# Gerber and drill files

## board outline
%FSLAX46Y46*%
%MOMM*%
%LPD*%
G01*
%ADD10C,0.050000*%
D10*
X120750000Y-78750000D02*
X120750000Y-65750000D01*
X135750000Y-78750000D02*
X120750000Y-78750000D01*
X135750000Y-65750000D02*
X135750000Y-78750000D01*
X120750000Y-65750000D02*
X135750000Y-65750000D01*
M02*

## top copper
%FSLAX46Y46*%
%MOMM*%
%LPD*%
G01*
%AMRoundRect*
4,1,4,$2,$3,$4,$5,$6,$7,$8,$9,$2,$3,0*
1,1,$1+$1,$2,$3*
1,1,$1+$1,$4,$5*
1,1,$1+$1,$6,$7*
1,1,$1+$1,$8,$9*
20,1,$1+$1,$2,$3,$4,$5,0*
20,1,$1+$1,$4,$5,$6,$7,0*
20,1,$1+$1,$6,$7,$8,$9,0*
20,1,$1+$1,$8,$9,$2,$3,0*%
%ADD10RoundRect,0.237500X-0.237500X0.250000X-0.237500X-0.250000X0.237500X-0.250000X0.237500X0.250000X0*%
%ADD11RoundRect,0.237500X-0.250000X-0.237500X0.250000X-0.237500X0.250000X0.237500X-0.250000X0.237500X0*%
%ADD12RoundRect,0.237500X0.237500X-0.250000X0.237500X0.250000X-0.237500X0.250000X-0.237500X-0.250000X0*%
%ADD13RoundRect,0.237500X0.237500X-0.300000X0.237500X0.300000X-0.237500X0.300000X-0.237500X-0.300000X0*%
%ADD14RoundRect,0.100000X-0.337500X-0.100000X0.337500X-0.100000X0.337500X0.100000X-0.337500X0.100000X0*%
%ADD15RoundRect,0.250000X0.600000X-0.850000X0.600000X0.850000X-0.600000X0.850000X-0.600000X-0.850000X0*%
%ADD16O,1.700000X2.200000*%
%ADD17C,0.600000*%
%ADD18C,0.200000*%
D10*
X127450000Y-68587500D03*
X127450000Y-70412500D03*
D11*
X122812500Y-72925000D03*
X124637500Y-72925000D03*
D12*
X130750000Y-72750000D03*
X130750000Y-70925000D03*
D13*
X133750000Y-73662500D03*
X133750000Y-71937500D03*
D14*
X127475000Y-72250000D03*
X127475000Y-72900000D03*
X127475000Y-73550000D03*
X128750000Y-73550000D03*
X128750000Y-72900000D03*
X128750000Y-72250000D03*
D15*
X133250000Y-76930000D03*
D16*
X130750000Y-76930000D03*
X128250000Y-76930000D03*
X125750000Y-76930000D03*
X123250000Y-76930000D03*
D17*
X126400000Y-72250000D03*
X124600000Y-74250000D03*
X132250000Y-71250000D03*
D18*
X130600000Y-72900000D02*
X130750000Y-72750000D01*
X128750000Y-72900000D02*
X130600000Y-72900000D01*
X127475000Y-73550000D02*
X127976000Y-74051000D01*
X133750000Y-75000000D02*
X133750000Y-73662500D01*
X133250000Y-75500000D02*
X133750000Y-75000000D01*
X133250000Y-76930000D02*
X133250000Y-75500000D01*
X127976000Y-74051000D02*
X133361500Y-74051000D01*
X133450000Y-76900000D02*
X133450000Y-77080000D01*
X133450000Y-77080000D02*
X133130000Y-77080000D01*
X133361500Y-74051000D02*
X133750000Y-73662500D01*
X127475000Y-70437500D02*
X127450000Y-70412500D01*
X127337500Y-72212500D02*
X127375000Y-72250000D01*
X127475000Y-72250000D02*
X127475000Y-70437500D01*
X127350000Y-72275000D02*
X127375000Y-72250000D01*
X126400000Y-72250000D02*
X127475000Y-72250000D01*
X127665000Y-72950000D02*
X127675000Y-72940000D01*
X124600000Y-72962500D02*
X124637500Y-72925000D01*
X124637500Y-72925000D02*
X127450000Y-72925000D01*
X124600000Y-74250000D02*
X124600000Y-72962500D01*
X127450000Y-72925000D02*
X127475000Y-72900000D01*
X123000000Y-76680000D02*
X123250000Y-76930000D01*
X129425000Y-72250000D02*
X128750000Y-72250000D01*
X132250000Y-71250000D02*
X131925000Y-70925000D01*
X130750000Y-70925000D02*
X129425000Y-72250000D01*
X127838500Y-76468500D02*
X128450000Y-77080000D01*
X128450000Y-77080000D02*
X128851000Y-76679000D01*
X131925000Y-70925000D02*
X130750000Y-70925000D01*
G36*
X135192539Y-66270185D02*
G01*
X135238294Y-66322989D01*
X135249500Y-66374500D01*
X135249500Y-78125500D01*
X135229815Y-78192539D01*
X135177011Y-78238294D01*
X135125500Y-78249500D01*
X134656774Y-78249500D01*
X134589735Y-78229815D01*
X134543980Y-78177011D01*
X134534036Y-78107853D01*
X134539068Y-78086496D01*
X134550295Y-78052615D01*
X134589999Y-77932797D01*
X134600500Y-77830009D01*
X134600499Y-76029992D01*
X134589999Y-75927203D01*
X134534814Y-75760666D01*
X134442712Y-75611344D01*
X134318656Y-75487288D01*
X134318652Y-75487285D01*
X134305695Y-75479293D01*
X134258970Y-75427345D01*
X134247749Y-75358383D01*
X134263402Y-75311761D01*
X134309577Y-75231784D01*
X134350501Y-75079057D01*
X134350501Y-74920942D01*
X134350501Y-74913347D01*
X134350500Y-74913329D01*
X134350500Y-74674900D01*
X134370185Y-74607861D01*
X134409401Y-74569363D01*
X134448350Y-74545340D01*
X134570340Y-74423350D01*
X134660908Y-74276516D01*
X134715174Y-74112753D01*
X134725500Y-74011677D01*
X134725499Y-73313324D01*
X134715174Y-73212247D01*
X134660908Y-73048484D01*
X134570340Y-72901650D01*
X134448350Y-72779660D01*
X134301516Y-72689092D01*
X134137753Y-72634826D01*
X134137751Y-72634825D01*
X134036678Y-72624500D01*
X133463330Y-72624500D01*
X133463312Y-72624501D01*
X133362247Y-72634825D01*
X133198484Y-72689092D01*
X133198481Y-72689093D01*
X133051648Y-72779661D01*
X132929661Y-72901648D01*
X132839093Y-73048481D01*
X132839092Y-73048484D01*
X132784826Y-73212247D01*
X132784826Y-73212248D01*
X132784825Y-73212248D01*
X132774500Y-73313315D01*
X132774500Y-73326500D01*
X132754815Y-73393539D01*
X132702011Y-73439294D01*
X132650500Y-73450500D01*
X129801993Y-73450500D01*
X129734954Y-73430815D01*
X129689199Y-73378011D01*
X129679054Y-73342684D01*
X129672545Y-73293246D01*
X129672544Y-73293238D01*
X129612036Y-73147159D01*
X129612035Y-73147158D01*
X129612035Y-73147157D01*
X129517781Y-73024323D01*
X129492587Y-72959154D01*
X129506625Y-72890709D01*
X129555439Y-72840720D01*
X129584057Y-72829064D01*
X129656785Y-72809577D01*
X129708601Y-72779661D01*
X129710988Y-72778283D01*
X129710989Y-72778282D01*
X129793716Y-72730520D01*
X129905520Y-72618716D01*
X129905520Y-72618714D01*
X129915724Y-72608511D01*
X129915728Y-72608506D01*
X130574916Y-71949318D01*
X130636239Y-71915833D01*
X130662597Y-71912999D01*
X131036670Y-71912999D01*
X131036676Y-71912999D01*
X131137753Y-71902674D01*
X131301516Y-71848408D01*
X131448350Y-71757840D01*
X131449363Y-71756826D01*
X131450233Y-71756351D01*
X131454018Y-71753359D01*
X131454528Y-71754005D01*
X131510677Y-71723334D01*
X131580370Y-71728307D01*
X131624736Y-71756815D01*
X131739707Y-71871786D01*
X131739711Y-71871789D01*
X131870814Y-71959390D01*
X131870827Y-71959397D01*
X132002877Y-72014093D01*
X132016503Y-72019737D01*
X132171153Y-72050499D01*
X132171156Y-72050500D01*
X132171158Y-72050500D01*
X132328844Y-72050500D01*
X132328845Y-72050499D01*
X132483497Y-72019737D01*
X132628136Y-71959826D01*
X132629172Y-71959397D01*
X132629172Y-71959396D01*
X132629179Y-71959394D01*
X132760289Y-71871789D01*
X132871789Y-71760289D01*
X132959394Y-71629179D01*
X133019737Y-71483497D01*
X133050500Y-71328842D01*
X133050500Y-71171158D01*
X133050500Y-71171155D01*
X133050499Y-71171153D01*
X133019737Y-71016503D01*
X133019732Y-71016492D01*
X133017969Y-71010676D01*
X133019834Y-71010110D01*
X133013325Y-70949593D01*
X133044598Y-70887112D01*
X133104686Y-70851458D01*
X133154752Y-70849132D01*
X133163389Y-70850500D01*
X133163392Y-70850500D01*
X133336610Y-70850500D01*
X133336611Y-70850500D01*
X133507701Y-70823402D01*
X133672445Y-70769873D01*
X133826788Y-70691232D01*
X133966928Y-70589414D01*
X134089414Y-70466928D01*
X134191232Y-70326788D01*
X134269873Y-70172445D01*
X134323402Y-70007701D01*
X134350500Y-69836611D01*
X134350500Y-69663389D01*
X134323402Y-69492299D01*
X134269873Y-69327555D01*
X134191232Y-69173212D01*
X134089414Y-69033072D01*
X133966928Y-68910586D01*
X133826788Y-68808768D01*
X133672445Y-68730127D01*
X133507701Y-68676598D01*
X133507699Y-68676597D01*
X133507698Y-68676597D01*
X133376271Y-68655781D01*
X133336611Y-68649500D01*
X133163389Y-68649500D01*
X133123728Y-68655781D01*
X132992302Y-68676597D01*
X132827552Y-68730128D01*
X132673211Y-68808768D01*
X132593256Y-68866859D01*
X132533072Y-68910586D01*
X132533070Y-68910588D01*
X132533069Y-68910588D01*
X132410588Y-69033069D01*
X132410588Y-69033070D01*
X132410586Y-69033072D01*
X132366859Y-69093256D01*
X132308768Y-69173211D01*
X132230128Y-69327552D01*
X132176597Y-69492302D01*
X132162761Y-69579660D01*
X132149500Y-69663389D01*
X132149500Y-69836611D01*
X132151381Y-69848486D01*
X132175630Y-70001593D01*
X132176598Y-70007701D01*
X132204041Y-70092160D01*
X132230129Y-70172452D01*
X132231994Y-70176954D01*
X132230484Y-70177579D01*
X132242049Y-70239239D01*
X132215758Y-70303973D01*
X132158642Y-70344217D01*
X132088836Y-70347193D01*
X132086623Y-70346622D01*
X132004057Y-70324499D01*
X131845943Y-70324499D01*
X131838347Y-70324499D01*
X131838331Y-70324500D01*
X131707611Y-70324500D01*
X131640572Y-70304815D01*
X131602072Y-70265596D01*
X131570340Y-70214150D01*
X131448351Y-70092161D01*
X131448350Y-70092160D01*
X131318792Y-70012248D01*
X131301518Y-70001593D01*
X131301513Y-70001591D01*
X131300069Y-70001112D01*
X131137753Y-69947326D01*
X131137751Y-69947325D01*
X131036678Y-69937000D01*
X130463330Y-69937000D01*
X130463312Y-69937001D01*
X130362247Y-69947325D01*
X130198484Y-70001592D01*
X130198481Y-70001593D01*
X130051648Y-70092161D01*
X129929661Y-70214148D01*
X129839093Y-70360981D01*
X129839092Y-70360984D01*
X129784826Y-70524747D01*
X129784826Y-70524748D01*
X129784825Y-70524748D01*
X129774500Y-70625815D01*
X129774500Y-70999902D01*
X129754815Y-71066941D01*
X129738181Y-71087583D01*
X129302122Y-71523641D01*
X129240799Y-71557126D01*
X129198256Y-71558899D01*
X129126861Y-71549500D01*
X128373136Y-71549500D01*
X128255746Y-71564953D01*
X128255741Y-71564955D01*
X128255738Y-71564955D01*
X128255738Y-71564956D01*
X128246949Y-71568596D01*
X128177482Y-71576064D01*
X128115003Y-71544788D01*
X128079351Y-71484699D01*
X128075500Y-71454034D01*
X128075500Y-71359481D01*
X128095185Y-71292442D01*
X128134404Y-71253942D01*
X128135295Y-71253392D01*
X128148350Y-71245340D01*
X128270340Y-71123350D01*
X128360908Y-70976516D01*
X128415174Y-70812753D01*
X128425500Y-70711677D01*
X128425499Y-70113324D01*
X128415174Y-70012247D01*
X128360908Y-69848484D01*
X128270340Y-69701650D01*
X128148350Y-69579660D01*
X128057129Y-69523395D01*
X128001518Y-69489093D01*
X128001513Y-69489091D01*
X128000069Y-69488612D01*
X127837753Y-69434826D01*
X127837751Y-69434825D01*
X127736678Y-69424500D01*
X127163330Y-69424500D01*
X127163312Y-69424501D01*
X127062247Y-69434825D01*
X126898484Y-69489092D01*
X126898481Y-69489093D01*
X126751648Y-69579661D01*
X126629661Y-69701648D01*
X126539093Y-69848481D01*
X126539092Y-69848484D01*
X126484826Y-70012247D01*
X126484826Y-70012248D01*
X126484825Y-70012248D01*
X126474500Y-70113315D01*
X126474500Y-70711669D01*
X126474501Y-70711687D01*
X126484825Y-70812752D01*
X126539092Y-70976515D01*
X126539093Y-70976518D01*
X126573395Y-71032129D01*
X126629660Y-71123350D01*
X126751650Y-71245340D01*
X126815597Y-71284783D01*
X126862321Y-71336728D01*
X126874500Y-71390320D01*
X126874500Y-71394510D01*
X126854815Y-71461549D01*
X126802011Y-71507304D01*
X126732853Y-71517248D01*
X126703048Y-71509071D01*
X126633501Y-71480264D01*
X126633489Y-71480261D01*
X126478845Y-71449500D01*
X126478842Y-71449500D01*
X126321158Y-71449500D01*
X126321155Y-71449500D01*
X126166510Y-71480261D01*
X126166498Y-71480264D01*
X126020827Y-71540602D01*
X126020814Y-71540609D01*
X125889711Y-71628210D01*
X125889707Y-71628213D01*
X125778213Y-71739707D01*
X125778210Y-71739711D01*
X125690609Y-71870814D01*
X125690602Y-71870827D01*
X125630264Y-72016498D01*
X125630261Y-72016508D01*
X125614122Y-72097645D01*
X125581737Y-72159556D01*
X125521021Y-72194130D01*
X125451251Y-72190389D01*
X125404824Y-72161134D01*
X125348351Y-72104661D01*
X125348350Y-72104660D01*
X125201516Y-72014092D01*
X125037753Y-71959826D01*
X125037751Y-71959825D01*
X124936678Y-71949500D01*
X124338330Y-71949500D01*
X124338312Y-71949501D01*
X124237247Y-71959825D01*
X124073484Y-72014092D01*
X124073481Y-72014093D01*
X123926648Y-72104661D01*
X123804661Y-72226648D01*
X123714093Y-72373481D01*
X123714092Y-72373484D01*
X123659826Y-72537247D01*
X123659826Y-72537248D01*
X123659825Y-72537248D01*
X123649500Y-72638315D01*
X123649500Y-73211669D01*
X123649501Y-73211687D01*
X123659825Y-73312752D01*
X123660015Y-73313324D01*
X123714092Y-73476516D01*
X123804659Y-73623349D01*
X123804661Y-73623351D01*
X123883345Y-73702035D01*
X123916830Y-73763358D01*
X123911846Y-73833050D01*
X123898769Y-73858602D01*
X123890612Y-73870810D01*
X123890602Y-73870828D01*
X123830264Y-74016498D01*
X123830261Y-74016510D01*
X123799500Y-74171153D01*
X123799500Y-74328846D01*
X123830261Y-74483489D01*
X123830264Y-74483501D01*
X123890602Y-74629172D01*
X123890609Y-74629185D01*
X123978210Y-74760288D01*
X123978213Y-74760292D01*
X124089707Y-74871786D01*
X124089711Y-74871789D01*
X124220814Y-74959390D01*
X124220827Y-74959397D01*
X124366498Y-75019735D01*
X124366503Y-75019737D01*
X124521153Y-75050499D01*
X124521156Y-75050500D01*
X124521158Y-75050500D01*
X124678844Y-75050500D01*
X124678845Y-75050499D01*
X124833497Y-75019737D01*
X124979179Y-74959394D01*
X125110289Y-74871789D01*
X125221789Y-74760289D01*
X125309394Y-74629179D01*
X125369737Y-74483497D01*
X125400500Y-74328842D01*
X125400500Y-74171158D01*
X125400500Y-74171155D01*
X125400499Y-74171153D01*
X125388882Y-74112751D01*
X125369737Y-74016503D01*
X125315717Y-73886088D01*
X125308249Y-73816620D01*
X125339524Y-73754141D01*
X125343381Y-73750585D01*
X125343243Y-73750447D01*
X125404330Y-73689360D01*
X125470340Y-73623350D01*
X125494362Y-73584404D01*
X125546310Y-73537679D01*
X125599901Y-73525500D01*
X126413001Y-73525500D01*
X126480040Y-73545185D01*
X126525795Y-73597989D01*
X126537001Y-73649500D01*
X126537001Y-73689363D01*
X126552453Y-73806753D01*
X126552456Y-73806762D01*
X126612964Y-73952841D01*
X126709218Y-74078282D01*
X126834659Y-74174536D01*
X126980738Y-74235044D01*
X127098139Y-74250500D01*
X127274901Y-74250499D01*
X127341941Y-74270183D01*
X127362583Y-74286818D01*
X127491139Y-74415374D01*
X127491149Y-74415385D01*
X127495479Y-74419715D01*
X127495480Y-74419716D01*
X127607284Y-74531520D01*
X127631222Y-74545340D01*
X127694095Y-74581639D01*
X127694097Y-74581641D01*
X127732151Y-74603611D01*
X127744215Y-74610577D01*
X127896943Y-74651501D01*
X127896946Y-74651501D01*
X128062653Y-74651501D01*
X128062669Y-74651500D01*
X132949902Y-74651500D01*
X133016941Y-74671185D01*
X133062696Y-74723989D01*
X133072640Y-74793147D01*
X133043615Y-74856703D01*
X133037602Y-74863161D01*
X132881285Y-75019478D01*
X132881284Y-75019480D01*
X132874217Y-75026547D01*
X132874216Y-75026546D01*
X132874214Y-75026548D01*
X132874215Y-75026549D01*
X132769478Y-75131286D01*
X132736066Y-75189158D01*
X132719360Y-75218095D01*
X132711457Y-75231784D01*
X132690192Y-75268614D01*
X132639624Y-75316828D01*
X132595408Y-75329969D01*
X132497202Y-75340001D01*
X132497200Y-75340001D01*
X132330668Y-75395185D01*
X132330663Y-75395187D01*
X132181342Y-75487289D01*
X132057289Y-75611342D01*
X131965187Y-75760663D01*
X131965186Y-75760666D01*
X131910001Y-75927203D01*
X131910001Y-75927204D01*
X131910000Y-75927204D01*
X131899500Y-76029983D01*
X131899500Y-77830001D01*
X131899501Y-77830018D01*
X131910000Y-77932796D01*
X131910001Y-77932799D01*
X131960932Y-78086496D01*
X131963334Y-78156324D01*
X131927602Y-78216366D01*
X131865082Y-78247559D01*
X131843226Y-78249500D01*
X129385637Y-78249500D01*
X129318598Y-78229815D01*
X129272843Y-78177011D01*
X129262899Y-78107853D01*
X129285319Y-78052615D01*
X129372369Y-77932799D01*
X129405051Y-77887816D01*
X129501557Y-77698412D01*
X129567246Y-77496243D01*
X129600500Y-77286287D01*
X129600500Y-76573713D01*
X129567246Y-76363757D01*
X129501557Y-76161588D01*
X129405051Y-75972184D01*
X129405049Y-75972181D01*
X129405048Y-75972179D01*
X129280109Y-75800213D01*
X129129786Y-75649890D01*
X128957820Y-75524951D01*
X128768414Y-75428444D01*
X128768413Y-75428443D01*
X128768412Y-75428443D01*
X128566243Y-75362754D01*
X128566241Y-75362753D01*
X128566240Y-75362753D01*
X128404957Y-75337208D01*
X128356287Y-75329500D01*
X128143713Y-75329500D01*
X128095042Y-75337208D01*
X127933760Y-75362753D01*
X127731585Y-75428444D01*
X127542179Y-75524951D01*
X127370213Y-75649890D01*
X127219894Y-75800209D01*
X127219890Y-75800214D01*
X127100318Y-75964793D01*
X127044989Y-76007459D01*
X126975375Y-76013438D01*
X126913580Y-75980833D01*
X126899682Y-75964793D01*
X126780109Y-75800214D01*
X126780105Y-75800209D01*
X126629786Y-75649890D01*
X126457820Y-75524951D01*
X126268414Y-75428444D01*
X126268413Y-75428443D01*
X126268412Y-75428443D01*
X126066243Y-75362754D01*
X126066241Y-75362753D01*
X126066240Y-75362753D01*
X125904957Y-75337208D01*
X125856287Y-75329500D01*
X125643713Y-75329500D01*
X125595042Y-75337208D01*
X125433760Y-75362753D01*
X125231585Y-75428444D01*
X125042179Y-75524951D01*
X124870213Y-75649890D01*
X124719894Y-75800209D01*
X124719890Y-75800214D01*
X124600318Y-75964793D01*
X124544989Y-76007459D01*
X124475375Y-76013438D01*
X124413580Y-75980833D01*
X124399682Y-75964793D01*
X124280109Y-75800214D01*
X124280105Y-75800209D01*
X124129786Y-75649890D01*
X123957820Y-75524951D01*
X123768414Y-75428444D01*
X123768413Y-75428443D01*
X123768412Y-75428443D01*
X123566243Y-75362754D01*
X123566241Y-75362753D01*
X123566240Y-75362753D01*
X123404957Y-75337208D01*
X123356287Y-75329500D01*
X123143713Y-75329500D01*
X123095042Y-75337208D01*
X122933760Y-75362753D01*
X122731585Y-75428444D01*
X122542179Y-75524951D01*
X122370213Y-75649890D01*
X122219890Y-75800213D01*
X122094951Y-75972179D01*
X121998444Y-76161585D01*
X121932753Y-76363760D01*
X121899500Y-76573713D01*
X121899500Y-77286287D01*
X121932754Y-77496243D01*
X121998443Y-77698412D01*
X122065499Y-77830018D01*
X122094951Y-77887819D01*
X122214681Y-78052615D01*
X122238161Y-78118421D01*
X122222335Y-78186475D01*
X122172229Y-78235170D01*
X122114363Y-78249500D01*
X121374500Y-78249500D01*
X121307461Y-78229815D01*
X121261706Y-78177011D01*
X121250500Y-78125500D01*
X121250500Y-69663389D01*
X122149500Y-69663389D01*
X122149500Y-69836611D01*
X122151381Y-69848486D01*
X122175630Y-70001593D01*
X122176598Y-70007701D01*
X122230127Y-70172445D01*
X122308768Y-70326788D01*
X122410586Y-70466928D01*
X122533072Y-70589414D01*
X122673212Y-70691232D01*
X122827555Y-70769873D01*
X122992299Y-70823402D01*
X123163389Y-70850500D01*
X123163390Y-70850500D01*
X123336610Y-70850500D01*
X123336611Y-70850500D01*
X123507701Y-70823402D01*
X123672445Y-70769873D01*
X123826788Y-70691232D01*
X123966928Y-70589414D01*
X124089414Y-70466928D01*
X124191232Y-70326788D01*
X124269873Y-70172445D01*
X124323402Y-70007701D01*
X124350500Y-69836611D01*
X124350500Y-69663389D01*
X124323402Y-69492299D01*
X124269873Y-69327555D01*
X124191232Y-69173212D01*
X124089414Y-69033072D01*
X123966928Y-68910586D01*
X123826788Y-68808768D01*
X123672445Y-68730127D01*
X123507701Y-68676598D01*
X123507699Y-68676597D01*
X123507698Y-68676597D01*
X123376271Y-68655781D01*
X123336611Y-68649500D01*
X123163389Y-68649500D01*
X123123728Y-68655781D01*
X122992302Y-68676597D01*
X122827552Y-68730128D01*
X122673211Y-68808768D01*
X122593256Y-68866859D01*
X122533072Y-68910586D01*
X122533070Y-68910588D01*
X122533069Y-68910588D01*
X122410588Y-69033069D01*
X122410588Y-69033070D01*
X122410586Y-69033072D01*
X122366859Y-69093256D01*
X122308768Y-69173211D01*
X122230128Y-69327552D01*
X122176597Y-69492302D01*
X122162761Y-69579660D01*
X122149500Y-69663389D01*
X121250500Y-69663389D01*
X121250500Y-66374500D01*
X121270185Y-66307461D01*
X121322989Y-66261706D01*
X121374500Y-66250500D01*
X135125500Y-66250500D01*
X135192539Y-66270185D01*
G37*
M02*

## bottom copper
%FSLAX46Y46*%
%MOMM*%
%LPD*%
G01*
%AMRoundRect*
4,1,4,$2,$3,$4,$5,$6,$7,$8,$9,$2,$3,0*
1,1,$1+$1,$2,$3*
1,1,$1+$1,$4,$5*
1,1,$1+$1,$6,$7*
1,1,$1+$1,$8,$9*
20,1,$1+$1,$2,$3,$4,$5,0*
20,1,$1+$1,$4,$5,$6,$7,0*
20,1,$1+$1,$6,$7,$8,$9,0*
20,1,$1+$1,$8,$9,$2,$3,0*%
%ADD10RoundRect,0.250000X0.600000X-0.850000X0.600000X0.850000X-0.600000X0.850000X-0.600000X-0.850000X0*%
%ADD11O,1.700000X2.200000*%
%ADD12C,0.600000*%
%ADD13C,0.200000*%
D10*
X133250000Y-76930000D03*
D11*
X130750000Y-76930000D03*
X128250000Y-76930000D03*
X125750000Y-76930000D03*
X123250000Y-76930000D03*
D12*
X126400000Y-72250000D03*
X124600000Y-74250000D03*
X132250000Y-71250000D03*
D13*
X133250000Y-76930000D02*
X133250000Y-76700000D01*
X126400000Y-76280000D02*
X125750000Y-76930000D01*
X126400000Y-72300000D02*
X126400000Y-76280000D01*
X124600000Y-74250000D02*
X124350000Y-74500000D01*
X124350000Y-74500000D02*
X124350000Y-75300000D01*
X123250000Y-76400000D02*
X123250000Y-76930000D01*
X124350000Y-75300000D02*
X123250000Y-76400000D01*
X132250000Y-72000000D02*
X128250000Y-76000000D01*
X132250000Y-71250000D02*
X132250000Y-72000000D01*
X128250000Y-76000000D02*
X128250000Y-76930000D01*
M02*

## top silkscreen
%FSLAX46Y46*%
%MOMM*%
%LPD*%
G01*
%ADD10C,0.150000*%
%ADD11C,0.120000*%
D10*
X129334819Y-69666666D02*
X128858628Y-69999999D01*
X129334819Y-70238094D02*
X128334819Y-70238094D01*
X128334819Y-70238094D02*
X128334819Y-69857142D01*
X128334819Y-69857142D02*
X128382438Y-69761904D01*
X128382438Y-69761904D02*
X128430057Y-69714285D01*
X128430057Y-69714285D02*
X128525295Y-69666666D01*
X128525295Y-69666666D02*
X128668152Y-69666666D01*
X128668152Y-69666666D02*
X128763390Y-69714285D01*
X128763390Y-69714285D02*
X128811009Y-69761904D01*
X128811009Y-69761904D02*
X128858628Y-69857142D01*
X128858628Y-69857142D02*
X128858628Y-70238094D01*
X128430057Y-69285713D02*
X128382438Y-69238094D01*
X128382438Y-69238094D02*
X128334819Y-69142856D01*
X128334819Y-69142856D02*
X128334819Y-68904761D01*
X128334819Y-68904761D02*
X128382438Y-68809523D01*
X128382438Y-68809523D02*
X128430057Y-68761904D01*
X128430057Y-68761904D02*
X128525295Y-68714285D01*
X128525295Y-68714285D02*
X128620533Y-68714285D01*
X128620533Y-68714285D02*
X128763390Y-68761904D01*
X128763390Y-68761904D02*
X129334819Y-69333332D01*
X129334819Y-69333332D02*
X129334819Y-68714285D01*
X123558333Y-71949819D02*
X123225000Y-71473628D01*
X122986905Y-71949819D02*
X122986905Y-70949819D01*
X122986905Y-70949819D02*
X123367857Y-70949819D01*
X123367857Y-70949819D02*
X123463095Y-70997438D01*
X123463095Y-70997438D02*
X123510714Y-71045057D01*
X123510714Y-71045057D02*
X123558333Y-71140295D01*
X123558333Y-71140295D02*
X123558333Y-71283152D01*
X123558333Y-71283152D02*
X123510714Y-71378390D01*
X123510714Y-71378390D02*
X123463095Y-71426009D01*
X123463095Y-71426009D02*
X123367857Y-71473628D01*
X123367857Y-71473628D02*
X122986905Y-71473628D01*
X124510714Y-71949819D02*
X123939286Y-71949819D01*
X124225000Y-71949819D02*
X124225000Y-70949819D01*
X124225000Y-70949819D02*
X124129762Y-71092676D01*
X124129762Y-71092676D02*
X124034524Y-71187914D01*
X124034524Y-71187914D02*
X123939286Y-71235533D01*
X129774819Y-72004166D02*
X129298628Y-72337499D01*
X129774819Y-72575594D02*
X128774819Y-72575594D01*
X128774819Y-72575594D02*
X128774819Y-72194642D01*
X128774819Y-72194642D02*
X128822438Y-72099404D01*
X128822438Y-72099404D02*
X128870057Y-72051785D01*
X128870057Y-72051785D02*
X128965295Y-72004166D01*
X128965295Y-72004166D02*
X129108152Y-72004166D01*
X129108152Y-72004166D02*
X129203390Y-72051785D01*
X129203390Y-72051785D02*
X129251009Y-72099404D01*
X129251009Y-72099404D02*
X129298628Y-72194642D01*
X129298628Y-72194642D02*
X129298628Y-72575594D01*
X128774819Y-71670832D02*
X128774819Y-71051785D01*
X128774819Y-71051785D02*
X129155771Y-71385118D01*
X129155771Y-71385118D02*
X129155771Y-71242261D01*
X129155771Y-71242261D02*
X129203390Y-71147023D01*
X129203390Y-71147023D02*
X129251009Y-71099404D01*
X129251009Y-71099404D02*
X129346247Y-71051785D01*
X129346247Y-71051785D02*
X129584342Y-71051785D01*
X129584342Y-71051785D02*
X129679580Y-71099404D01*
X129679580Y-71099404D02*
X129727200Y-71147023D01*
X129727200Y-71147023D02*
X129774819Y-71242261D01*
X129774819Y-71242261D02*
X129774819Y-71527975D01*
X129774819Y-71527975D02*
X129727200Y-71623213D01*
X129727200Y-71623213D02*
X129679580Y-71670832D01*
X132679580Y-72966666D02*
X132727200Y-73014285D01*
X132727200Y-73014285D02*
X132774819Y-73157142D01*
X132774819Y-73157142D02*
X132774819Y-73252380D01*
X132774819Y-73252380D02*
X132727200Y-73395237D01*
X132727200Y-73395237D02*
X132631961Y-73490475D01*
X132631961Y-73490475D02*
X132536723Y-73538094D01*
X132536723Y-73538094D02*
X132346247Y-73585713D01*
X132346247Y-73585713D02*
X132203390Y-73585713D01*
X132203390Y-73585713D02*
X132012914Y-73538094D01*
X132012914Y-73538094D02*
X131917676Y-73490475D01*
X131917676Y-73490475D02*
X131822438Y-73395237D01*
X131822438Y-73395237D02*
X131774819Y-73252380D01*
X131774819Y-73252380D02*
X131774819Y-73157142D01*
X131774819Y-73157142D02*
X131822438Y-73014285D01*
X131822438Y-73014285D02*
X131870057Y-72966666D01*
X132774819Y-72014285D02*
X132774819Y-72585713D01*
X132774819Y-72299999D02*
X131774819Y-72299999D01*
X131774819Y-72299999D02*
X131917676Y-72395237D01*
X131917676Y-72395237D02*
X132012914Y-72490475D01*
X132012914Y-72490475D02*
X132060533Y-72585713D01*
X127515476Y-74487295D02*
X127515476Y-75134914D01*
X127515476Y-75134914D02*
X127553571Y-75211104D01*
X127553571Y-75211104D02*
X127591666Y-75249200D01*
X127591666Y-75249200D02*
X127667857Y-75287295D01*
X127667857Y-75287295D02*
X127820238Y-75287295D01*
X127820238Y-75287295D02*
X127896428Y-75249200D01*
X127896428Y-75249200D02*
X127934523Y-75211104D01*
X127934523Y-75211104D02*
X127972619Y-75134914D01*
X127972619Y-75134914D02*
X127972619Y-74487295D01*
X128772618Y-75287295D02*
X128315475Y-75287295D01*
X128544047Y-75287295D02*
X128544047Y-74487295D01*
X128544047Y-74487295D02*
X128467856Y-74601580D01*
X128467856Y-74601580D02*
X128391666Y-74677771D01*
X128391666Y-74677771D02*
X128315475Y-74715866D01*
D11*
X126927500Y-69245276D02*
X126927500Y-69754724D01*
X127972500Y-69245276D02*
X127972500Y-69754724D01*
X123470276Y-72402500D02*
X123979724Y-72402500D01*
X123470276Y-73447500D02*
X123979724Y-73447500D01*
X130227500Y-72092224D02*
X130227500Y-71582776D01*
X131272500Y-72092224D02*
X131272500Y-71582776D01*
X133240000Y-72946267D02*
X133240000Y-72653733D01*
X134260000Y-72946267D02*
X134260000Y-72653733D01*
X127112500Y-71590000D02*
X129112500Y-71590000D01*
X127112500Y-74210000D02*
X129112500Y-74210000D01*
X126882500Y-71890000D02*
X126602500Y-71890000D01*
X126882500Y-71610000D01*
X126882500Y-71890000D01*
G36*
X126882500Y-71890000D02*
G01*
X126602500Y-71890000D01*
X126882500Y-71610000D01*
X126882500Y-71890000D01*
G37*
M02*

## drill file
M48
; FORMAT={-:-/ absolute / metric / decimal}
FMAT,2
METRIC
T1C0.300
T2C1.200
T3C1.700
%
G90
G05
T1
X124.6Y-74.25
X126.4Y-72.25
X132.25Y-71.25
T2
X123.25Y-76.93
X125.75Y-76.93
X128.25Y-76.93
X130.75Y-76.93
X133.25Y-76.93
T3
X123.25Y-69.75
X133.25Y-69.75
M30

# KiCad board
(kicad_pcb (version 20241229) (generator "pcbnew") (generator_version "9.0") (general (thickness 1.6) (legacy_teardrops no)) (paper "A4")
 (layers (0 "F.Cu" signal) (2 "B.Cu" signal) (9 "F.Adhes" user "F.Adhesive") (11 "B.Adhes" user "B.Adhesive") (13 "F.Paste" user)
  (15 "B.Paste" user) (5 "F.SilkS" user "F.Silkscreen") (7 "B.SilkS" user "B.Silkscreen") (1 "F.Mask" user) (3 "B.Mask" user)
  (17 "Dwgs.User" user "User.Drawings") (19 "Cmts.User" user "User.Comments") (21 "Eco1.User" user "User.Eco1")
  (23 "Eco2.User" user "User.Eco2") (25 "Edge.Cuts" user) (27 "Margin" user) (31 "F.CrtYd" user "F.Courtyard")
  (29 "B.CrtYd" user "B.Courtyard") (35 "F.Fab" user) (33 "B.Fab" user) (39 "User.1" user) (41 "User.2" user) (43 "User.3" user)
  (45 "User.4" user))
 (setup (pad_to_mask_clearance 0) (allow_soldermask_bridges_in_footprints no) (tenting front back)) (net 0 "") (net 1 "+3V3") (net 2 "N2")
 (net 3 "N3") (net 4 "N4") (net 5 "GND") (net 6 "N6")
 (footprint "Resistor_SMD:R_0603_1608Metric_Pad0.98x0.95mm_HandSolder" (layer "F.Cu") (at 127.45 69.5 -90)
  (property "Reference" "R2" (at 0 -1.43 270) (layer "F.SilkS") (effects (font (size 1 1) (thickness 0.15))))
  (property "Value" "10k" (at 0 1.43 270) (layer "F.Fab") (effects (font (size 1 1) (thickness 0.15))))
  (fp_line (start -0.254724 0.5225) (end 0.254724 0.5225) (stroke (width 0.12) (type solid)) (layer "F.SilkS"))
  (fp_line (start -0.254724 -0.5225) (end 0.254724 -0.5225) (stroke (width 0.12) (type solid)) (layer "F.SilkS"))
  (pad "1" smd roundrect (at -0.9125 0 270) (size 0.975 0.95) (layers "F.Cu" "F.Mask" "F.Paste") (roundrect_rratio 0.25) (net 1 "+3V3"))
  (pad "2" smd roundrect (at 0.9125 0 270) (size 0.975 0.95) (layers "F.Cu" "F.Mask" "F.Paste") (roundrect_rratio 0.25) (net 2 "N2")))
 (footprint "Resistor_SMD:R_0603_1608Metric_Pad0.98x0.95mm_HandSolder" (layer "F.Cu") (at 123.725 72.925)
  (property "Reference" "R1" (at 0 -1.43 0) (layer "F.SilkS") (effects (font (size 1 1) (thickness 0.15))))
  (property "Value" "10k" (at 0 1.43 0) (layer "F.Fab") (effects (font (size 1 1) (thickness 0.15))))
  (fp_line (start -0.254724 -0.5225) (end 0.254724 -0.5225) (stroke (width 0.12) (type solid)) (layer "F.SilkS"))
  (fp_line (start -0.254724 0.5225) (end 0.254724 0.5225) (stroke (width 0.12) (type solid)) (layer "F.SilkS"))
  (pad "1" smd roundrect (at -0.9125 0) (size 0.975 0.95) (layers "F.Cu" "F.Mask" "F.Paste") (roundrect_rratio 0.25) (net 1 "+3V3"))
  (pad "2" smd roundrect (at 0.9125 0) (size 0.975 0.95) (layers "F.Cu" "F.Mask" "F.Paste") (roundrect_rratio 0.25) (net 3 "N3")))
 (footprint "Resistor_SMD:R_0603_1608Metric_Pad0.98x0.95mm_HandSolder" (layer "F.Cu") (at 130.75 71.8375 90)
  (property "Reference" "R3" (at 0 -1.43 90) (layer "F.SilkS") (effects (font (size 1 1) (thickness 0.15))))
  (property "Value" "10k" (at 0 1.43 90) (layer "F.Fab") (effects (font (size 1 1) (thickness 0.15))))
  (fp_line (start -0.254724 -0.5225) (end 0.254724 -0.5225) (stroke (width 0.12) (type solid)) (layer "F.SilkS"))
  (fp_line (start -0.254724 0.5225) (end 0.254724 0.5225) (stroke (width 0.12) (type solid)) (layer "F.SilkS"))
  (pad "1" smd roundrect (at -0.9125 0 90) (size 0.975 0.95) (layers "F.Cu" "F.Mask" "F.Paste") (roundrect_rratio 0.25) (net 1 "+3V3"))
  (pad "2" smd roundrect (at 0.9125 0 90) (size 0.975 0.95) (layers "F.Cu" "F.Mask" "F.Paste") (roundrect_rratio 0.25) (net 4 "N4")))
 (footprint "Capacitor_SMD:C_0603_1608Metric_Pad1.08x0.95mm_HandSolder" (layer "F.Cu") (at 133.75 72.8 90)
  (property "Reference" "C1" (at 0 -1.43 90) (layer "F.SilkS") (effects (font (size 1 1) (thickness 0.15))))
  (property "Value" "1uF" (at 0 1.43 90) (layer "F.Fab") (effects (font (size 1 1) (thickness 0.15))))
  (fp_line (start -0.146267 -0.51) (end 0.146267 -0.51) (stroke (width 0.12) (type solid)) (layer "F.SilkS"))
  (fp_line (start -0.146267 0.51) (end 0.146267 0.51) (stroke (width 0.12) (type solid)) (layer "F.SilkS"))
  (pad "1" smd roundrect (at -0.8625 0 90) (size 1.075 0.95) (layers "F.Cu" "F.Mask" "F.Paste") (roundrect_rratio 0.25) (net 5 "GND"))
  (pad "2" smd roundrect (at 0.8625 0 90) (size 1.075 0.95) (layers "F.Cu" "F.Mask" "F.Paste") (roundrect_rratio 0.25) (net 1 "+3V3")))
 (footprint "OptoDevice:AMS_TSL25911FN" (layer "F.Cu") (at 128.1125 72.9)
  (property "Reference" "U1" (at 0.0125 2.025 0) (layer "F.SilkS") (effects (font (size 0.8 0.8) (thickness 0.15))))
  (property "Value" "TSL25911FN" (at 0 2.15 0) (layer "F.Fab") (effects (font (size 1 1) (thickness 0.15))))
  (fp_line (start -1 -1.31) (end 1 -1.31) (stroke (width 0.12) (type solid)) (layer "F.SilkS"))
  (fp_line (start -1 1.31) (end 1 1.31) (stroke (width 0.12) (type solid)) (layer "F.SilkS"))
  (fp_poly
   (pts (xy -1.23 -1.01) (xy -1.51 -1.01) (xy -1.23 -1.29) (xy -1.23 -1.01)) (stroke (width 0.12) (type solid)) (fill yes) (layer "F.SilkS"))
  (pad "1" smd roundrect (at -0.6375 -0.65) (size 0.875 0.4) (layers "F.Cu" "F.Mask" "F.Paste") (roundrect_rratio 0.25) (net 2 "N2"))
  (pad "2" smd roundrect (at -0.6375 0) (size 0.875 0.4) (layers "F.Cu" "F.Mask" "F.Paste") (roundrect_rratio 0.25) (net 3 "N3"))
  (pad "3" smd roundrect (at -0.6375 0.65) (size 0.875 0.4) (layers "F.Cu" "F.Mask" "F.Paste") (roundrect_rratio 0.25) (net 5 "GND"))
  (pad "4" smd roundrect (at 0.6375 0.65) (size 0.875 0.4) (layers "F.Cu" "F.Mask" "F.Paste") (roundrect_rratio 0.25) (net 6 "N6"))
  (pad "5" smd roundrect (at 0.6375 0) (size 0.875 0.4) (layers "F.Cu" "F.Mask" "F.Paste") (roundrect_rratio 0.25) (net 1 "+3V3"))
  (pad "6" smd roundrect (at 0.6375 -0.65) (size 0.875 0.4) (layers "F.Cu" "F.Mask" "F.Paste") (roundrect_rratio 0.25) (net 4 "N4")))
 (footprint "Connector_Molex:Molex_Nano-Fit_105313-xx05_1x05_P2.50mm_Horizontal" (layer "B.Cu") (at 133.25 76.93 90)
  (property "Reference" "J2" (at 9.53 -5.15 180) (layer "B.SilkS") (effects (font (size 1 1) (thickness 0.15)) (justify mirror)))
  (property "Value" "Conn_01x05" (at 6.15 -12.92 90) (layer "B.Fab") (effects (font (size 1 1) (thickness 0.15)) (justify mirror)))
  (pad "" np_thru_hole circle (at 7.18 -10 90) (size 1.7 1.7) (drill 1.7) (layers "*.Cu" "*.Mask"))
  (pad "" np_thru_hole circle (at 7.18 0 90) (size 1.7 1.7) (drill 1.7) (layers "*.Cu" "*.Mask"))
  (pad "1" thru_hole roundrect (at 0 0 90) (size 2.2 1.7) (drill 1.2) (layers "*.Cu" "*.Mask") (remove_unused_layers no)
   (roundrect_rratio 0.147059) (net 5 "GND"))
  (pad "2" thru_hole oval (at 0 -2.5 90) (size 2.2 1.7) (drill 1.2) (layers "*.Cu" "*.Mask") (remove_unused_layers no) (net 1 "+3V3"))
  (pad "3" thru_hole oval (at 0 -5 90) (size 2.2 1.7) (drill 1.2) (layers "*.Cu" "*.Mask") (remove_unused_layers no) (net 4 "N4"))
  (pad "4" thru_hole oval (at 0 -7.5 90) (size 2.2 1.7) (drill 1.2) (layers "*.Cu" "*.Mask") (remove_unused_layers no) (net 2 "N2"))
  (pad "5" thru_hole oval (at 0 -10 90) (size 2.2 1.7) (drill 1.2) (layers "*.Cu" "*.Mask") (remove_unused_layers no) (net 3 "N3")))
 (gr_line (start 120.75 78.75) (end 120.75 65.75) (stroke (width 0.05) (type default)) (layer "Edge.Cuts"))
 (gr_line (start 135.75 78.75) (end 120.75 78.75) (stroke (width 0.05) (type default)) (layer "Edge.Cuts"))
 (gr_line (start 135.75 65.75) (end 135.75 78.75) (stroke (width 0.05) (type default)) (layer "Edge.Cuts"))
 (gr_line (start 120.75 65.75) (end 135.75 65.75) (stroke (width 0.05) (type default)) (layer "Edge.Cuts"))
 (segment (start 130.6 72.9) (end 130.75 72.75) (width 0.2) (layer "F.Cu") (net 1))
 (segment (start 128.75 72.9) (end 130.6 72.9) (width 0.2) (layer "F.Cu") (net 1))
 (segment (start 127.475 73.55) (end 127.976 74.051) (width 0.2) (layer "F.Cu") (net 5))
 (segment (start 133.75 75) (end 133.75 73.6625) (width 0.2) (layer "F.Cu") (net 5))
 (segment (start 133.25 75.5) (end 133.75 75) (width 0.2) (layer "F.Cu") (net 5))
 (segment (start 133.25 76.93) (end 133.25 75.5) (width 0.2) (layer "F.Cu") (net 5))
 (segment (start 127.976 74.051) (end 133.3615 74.051) (width 0.2) (layer "F.Cu") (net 5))
 (segment (start 133.45 76.9) (end 133.45 77.08) (width 0.2) (layer "F.Cu") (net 5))
 (segment (start 133.45 77.08) (end 133.13 77.08) (width 0.2) (layer "F.Cu") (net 5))
 (segment (start 133.3615 74.051) (end 133.75 73.6625) (width 0.2) (layer "F.Cu") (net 5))
 (segment (start 133.25 76.93) (end 133.25 76.7) (width 0.2) (layer "B.Cu") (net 5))
 (segment (start 127.475 70.4375) (end 127.45 70.4125) (width 0.2) (layer "F.Cu") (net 2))
 (segment (start 127.3375 72.2125) (end 127.375 72.25) (width 0.2) (layer "F.Cu") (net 2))
 (segment (start 127.475 72.25) (end 127.475 70.4375) (width 0.2) (layer "F.Cu") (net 2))
 (segment (start 127.35 72.275) (end 127.375 72.25) (width 0.2) (layer "F.Cu") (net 2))
 (segment (start 126.4 72.25) (end 127.475 72.25) (width 0.2) (layer "F.Cu") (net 2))
 (via (at 126.4 72.25) (size 0.6) (drill 0.3) (layers "F.Cu" "B.Cu") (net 2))
 (segment (start 126.4 76.28) (end 125.75 76.93) (width 0.2) (layer "B.Cu") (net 2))
 (segment (start 126.4 72.3) (end 126.4 76.28) (width 0.2) (layer "B.Cu") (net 2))
 (segment (start 127.665 72.95) (end 127.675 72.94) (width 0.2) (layer "F.Cu") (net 3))
 (segment (start 124.6 72.9625) (end 124.6375 72.925) (width 0.2) (layer "F.Cu") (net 3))
 (segment (start 124.6375 72.925) (end 127.45 72.925) (width 0.2) (layer "F.Cu") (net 3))
 (segment (start 124.6 74.25) (end 124.6 72.9625) (width 0.2) (layer "F.Cu") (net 3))
 (segment (start 127.45 72.925) (end 127.475 72.9) (width 0.2) (layer "F.Cu") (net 3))
 (segment (start 123 76.68) (end 123.25 76.93) (width 0.2) (layer "F.Cu") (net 3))
 (via (at 124.6 74.25) (size 0.6) (drill 0.3) (layers "F.Cu" "B.Cu") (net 3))
 (segment (start 124.6 74.25) (end 124.35 74.5) (width 0.2) (layer "B.Cu") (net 3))
 (segment (start 124.35 74.5) (end 124.35 75.3) (width 0.2) (layer "B.Cu") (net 3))
 (segment (start 123.25 76.4) (end 123.25 76.93) (width 0.2) (layer "B.Cu") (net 3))
 (segment (start 124.35 75.3) (end 123.25 76.4) (width 0.2) (layer "B.Cu") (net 3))
 (segment (start 129.425 72.25) (end 128.75 72.25) (width 0.2) (layer "F.Cu") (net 4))
 (segment (start 132.25 71.25) (end 131.925 70.925) (width 0.2) (layer "F.Cu") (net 4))
 (segment (start 130.75 70.925) (end 129.425 72.25) (width 0.2) (layer "F.Cu") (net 4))
 (segment (start 127.8385 76.4685) (end 128.45 77.08) (width 0.2) (layer "F.Cu") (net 4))
 (segment (start 128.45 77.08) (end 128.851 76.679) (width 0.2) (layer "F.Cu") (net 4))
 (segment (start 131.925 70.925) (end 130.75 70.925) (width 0.2) (layer "F.Cu") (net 4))
 (via (at 132.25 71.25) (size 0.6) (drill 0.3) (layers "F.Cu" "B.Cu") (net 4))
 (segment (start 132.25 72) (end 128.25 76) (width 0.2) (layer "B.Cu") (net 4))
 (segment (start 132.25 71.25) (end 132.25 72) (width 0.2) (layer "B.Cu") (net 4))
 (segment (start 128.25 76) (end 128.25 76.93) (width 0.2) (layer "B.Cu") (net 4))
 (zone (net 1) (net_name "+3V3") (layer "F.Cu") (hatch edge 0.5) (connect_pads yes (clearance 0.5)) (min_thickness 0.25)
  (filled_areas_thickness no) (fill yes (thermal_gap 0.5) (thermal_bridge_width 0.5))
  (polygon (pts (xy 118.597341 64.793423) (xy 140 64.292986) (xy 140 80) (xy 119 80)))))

